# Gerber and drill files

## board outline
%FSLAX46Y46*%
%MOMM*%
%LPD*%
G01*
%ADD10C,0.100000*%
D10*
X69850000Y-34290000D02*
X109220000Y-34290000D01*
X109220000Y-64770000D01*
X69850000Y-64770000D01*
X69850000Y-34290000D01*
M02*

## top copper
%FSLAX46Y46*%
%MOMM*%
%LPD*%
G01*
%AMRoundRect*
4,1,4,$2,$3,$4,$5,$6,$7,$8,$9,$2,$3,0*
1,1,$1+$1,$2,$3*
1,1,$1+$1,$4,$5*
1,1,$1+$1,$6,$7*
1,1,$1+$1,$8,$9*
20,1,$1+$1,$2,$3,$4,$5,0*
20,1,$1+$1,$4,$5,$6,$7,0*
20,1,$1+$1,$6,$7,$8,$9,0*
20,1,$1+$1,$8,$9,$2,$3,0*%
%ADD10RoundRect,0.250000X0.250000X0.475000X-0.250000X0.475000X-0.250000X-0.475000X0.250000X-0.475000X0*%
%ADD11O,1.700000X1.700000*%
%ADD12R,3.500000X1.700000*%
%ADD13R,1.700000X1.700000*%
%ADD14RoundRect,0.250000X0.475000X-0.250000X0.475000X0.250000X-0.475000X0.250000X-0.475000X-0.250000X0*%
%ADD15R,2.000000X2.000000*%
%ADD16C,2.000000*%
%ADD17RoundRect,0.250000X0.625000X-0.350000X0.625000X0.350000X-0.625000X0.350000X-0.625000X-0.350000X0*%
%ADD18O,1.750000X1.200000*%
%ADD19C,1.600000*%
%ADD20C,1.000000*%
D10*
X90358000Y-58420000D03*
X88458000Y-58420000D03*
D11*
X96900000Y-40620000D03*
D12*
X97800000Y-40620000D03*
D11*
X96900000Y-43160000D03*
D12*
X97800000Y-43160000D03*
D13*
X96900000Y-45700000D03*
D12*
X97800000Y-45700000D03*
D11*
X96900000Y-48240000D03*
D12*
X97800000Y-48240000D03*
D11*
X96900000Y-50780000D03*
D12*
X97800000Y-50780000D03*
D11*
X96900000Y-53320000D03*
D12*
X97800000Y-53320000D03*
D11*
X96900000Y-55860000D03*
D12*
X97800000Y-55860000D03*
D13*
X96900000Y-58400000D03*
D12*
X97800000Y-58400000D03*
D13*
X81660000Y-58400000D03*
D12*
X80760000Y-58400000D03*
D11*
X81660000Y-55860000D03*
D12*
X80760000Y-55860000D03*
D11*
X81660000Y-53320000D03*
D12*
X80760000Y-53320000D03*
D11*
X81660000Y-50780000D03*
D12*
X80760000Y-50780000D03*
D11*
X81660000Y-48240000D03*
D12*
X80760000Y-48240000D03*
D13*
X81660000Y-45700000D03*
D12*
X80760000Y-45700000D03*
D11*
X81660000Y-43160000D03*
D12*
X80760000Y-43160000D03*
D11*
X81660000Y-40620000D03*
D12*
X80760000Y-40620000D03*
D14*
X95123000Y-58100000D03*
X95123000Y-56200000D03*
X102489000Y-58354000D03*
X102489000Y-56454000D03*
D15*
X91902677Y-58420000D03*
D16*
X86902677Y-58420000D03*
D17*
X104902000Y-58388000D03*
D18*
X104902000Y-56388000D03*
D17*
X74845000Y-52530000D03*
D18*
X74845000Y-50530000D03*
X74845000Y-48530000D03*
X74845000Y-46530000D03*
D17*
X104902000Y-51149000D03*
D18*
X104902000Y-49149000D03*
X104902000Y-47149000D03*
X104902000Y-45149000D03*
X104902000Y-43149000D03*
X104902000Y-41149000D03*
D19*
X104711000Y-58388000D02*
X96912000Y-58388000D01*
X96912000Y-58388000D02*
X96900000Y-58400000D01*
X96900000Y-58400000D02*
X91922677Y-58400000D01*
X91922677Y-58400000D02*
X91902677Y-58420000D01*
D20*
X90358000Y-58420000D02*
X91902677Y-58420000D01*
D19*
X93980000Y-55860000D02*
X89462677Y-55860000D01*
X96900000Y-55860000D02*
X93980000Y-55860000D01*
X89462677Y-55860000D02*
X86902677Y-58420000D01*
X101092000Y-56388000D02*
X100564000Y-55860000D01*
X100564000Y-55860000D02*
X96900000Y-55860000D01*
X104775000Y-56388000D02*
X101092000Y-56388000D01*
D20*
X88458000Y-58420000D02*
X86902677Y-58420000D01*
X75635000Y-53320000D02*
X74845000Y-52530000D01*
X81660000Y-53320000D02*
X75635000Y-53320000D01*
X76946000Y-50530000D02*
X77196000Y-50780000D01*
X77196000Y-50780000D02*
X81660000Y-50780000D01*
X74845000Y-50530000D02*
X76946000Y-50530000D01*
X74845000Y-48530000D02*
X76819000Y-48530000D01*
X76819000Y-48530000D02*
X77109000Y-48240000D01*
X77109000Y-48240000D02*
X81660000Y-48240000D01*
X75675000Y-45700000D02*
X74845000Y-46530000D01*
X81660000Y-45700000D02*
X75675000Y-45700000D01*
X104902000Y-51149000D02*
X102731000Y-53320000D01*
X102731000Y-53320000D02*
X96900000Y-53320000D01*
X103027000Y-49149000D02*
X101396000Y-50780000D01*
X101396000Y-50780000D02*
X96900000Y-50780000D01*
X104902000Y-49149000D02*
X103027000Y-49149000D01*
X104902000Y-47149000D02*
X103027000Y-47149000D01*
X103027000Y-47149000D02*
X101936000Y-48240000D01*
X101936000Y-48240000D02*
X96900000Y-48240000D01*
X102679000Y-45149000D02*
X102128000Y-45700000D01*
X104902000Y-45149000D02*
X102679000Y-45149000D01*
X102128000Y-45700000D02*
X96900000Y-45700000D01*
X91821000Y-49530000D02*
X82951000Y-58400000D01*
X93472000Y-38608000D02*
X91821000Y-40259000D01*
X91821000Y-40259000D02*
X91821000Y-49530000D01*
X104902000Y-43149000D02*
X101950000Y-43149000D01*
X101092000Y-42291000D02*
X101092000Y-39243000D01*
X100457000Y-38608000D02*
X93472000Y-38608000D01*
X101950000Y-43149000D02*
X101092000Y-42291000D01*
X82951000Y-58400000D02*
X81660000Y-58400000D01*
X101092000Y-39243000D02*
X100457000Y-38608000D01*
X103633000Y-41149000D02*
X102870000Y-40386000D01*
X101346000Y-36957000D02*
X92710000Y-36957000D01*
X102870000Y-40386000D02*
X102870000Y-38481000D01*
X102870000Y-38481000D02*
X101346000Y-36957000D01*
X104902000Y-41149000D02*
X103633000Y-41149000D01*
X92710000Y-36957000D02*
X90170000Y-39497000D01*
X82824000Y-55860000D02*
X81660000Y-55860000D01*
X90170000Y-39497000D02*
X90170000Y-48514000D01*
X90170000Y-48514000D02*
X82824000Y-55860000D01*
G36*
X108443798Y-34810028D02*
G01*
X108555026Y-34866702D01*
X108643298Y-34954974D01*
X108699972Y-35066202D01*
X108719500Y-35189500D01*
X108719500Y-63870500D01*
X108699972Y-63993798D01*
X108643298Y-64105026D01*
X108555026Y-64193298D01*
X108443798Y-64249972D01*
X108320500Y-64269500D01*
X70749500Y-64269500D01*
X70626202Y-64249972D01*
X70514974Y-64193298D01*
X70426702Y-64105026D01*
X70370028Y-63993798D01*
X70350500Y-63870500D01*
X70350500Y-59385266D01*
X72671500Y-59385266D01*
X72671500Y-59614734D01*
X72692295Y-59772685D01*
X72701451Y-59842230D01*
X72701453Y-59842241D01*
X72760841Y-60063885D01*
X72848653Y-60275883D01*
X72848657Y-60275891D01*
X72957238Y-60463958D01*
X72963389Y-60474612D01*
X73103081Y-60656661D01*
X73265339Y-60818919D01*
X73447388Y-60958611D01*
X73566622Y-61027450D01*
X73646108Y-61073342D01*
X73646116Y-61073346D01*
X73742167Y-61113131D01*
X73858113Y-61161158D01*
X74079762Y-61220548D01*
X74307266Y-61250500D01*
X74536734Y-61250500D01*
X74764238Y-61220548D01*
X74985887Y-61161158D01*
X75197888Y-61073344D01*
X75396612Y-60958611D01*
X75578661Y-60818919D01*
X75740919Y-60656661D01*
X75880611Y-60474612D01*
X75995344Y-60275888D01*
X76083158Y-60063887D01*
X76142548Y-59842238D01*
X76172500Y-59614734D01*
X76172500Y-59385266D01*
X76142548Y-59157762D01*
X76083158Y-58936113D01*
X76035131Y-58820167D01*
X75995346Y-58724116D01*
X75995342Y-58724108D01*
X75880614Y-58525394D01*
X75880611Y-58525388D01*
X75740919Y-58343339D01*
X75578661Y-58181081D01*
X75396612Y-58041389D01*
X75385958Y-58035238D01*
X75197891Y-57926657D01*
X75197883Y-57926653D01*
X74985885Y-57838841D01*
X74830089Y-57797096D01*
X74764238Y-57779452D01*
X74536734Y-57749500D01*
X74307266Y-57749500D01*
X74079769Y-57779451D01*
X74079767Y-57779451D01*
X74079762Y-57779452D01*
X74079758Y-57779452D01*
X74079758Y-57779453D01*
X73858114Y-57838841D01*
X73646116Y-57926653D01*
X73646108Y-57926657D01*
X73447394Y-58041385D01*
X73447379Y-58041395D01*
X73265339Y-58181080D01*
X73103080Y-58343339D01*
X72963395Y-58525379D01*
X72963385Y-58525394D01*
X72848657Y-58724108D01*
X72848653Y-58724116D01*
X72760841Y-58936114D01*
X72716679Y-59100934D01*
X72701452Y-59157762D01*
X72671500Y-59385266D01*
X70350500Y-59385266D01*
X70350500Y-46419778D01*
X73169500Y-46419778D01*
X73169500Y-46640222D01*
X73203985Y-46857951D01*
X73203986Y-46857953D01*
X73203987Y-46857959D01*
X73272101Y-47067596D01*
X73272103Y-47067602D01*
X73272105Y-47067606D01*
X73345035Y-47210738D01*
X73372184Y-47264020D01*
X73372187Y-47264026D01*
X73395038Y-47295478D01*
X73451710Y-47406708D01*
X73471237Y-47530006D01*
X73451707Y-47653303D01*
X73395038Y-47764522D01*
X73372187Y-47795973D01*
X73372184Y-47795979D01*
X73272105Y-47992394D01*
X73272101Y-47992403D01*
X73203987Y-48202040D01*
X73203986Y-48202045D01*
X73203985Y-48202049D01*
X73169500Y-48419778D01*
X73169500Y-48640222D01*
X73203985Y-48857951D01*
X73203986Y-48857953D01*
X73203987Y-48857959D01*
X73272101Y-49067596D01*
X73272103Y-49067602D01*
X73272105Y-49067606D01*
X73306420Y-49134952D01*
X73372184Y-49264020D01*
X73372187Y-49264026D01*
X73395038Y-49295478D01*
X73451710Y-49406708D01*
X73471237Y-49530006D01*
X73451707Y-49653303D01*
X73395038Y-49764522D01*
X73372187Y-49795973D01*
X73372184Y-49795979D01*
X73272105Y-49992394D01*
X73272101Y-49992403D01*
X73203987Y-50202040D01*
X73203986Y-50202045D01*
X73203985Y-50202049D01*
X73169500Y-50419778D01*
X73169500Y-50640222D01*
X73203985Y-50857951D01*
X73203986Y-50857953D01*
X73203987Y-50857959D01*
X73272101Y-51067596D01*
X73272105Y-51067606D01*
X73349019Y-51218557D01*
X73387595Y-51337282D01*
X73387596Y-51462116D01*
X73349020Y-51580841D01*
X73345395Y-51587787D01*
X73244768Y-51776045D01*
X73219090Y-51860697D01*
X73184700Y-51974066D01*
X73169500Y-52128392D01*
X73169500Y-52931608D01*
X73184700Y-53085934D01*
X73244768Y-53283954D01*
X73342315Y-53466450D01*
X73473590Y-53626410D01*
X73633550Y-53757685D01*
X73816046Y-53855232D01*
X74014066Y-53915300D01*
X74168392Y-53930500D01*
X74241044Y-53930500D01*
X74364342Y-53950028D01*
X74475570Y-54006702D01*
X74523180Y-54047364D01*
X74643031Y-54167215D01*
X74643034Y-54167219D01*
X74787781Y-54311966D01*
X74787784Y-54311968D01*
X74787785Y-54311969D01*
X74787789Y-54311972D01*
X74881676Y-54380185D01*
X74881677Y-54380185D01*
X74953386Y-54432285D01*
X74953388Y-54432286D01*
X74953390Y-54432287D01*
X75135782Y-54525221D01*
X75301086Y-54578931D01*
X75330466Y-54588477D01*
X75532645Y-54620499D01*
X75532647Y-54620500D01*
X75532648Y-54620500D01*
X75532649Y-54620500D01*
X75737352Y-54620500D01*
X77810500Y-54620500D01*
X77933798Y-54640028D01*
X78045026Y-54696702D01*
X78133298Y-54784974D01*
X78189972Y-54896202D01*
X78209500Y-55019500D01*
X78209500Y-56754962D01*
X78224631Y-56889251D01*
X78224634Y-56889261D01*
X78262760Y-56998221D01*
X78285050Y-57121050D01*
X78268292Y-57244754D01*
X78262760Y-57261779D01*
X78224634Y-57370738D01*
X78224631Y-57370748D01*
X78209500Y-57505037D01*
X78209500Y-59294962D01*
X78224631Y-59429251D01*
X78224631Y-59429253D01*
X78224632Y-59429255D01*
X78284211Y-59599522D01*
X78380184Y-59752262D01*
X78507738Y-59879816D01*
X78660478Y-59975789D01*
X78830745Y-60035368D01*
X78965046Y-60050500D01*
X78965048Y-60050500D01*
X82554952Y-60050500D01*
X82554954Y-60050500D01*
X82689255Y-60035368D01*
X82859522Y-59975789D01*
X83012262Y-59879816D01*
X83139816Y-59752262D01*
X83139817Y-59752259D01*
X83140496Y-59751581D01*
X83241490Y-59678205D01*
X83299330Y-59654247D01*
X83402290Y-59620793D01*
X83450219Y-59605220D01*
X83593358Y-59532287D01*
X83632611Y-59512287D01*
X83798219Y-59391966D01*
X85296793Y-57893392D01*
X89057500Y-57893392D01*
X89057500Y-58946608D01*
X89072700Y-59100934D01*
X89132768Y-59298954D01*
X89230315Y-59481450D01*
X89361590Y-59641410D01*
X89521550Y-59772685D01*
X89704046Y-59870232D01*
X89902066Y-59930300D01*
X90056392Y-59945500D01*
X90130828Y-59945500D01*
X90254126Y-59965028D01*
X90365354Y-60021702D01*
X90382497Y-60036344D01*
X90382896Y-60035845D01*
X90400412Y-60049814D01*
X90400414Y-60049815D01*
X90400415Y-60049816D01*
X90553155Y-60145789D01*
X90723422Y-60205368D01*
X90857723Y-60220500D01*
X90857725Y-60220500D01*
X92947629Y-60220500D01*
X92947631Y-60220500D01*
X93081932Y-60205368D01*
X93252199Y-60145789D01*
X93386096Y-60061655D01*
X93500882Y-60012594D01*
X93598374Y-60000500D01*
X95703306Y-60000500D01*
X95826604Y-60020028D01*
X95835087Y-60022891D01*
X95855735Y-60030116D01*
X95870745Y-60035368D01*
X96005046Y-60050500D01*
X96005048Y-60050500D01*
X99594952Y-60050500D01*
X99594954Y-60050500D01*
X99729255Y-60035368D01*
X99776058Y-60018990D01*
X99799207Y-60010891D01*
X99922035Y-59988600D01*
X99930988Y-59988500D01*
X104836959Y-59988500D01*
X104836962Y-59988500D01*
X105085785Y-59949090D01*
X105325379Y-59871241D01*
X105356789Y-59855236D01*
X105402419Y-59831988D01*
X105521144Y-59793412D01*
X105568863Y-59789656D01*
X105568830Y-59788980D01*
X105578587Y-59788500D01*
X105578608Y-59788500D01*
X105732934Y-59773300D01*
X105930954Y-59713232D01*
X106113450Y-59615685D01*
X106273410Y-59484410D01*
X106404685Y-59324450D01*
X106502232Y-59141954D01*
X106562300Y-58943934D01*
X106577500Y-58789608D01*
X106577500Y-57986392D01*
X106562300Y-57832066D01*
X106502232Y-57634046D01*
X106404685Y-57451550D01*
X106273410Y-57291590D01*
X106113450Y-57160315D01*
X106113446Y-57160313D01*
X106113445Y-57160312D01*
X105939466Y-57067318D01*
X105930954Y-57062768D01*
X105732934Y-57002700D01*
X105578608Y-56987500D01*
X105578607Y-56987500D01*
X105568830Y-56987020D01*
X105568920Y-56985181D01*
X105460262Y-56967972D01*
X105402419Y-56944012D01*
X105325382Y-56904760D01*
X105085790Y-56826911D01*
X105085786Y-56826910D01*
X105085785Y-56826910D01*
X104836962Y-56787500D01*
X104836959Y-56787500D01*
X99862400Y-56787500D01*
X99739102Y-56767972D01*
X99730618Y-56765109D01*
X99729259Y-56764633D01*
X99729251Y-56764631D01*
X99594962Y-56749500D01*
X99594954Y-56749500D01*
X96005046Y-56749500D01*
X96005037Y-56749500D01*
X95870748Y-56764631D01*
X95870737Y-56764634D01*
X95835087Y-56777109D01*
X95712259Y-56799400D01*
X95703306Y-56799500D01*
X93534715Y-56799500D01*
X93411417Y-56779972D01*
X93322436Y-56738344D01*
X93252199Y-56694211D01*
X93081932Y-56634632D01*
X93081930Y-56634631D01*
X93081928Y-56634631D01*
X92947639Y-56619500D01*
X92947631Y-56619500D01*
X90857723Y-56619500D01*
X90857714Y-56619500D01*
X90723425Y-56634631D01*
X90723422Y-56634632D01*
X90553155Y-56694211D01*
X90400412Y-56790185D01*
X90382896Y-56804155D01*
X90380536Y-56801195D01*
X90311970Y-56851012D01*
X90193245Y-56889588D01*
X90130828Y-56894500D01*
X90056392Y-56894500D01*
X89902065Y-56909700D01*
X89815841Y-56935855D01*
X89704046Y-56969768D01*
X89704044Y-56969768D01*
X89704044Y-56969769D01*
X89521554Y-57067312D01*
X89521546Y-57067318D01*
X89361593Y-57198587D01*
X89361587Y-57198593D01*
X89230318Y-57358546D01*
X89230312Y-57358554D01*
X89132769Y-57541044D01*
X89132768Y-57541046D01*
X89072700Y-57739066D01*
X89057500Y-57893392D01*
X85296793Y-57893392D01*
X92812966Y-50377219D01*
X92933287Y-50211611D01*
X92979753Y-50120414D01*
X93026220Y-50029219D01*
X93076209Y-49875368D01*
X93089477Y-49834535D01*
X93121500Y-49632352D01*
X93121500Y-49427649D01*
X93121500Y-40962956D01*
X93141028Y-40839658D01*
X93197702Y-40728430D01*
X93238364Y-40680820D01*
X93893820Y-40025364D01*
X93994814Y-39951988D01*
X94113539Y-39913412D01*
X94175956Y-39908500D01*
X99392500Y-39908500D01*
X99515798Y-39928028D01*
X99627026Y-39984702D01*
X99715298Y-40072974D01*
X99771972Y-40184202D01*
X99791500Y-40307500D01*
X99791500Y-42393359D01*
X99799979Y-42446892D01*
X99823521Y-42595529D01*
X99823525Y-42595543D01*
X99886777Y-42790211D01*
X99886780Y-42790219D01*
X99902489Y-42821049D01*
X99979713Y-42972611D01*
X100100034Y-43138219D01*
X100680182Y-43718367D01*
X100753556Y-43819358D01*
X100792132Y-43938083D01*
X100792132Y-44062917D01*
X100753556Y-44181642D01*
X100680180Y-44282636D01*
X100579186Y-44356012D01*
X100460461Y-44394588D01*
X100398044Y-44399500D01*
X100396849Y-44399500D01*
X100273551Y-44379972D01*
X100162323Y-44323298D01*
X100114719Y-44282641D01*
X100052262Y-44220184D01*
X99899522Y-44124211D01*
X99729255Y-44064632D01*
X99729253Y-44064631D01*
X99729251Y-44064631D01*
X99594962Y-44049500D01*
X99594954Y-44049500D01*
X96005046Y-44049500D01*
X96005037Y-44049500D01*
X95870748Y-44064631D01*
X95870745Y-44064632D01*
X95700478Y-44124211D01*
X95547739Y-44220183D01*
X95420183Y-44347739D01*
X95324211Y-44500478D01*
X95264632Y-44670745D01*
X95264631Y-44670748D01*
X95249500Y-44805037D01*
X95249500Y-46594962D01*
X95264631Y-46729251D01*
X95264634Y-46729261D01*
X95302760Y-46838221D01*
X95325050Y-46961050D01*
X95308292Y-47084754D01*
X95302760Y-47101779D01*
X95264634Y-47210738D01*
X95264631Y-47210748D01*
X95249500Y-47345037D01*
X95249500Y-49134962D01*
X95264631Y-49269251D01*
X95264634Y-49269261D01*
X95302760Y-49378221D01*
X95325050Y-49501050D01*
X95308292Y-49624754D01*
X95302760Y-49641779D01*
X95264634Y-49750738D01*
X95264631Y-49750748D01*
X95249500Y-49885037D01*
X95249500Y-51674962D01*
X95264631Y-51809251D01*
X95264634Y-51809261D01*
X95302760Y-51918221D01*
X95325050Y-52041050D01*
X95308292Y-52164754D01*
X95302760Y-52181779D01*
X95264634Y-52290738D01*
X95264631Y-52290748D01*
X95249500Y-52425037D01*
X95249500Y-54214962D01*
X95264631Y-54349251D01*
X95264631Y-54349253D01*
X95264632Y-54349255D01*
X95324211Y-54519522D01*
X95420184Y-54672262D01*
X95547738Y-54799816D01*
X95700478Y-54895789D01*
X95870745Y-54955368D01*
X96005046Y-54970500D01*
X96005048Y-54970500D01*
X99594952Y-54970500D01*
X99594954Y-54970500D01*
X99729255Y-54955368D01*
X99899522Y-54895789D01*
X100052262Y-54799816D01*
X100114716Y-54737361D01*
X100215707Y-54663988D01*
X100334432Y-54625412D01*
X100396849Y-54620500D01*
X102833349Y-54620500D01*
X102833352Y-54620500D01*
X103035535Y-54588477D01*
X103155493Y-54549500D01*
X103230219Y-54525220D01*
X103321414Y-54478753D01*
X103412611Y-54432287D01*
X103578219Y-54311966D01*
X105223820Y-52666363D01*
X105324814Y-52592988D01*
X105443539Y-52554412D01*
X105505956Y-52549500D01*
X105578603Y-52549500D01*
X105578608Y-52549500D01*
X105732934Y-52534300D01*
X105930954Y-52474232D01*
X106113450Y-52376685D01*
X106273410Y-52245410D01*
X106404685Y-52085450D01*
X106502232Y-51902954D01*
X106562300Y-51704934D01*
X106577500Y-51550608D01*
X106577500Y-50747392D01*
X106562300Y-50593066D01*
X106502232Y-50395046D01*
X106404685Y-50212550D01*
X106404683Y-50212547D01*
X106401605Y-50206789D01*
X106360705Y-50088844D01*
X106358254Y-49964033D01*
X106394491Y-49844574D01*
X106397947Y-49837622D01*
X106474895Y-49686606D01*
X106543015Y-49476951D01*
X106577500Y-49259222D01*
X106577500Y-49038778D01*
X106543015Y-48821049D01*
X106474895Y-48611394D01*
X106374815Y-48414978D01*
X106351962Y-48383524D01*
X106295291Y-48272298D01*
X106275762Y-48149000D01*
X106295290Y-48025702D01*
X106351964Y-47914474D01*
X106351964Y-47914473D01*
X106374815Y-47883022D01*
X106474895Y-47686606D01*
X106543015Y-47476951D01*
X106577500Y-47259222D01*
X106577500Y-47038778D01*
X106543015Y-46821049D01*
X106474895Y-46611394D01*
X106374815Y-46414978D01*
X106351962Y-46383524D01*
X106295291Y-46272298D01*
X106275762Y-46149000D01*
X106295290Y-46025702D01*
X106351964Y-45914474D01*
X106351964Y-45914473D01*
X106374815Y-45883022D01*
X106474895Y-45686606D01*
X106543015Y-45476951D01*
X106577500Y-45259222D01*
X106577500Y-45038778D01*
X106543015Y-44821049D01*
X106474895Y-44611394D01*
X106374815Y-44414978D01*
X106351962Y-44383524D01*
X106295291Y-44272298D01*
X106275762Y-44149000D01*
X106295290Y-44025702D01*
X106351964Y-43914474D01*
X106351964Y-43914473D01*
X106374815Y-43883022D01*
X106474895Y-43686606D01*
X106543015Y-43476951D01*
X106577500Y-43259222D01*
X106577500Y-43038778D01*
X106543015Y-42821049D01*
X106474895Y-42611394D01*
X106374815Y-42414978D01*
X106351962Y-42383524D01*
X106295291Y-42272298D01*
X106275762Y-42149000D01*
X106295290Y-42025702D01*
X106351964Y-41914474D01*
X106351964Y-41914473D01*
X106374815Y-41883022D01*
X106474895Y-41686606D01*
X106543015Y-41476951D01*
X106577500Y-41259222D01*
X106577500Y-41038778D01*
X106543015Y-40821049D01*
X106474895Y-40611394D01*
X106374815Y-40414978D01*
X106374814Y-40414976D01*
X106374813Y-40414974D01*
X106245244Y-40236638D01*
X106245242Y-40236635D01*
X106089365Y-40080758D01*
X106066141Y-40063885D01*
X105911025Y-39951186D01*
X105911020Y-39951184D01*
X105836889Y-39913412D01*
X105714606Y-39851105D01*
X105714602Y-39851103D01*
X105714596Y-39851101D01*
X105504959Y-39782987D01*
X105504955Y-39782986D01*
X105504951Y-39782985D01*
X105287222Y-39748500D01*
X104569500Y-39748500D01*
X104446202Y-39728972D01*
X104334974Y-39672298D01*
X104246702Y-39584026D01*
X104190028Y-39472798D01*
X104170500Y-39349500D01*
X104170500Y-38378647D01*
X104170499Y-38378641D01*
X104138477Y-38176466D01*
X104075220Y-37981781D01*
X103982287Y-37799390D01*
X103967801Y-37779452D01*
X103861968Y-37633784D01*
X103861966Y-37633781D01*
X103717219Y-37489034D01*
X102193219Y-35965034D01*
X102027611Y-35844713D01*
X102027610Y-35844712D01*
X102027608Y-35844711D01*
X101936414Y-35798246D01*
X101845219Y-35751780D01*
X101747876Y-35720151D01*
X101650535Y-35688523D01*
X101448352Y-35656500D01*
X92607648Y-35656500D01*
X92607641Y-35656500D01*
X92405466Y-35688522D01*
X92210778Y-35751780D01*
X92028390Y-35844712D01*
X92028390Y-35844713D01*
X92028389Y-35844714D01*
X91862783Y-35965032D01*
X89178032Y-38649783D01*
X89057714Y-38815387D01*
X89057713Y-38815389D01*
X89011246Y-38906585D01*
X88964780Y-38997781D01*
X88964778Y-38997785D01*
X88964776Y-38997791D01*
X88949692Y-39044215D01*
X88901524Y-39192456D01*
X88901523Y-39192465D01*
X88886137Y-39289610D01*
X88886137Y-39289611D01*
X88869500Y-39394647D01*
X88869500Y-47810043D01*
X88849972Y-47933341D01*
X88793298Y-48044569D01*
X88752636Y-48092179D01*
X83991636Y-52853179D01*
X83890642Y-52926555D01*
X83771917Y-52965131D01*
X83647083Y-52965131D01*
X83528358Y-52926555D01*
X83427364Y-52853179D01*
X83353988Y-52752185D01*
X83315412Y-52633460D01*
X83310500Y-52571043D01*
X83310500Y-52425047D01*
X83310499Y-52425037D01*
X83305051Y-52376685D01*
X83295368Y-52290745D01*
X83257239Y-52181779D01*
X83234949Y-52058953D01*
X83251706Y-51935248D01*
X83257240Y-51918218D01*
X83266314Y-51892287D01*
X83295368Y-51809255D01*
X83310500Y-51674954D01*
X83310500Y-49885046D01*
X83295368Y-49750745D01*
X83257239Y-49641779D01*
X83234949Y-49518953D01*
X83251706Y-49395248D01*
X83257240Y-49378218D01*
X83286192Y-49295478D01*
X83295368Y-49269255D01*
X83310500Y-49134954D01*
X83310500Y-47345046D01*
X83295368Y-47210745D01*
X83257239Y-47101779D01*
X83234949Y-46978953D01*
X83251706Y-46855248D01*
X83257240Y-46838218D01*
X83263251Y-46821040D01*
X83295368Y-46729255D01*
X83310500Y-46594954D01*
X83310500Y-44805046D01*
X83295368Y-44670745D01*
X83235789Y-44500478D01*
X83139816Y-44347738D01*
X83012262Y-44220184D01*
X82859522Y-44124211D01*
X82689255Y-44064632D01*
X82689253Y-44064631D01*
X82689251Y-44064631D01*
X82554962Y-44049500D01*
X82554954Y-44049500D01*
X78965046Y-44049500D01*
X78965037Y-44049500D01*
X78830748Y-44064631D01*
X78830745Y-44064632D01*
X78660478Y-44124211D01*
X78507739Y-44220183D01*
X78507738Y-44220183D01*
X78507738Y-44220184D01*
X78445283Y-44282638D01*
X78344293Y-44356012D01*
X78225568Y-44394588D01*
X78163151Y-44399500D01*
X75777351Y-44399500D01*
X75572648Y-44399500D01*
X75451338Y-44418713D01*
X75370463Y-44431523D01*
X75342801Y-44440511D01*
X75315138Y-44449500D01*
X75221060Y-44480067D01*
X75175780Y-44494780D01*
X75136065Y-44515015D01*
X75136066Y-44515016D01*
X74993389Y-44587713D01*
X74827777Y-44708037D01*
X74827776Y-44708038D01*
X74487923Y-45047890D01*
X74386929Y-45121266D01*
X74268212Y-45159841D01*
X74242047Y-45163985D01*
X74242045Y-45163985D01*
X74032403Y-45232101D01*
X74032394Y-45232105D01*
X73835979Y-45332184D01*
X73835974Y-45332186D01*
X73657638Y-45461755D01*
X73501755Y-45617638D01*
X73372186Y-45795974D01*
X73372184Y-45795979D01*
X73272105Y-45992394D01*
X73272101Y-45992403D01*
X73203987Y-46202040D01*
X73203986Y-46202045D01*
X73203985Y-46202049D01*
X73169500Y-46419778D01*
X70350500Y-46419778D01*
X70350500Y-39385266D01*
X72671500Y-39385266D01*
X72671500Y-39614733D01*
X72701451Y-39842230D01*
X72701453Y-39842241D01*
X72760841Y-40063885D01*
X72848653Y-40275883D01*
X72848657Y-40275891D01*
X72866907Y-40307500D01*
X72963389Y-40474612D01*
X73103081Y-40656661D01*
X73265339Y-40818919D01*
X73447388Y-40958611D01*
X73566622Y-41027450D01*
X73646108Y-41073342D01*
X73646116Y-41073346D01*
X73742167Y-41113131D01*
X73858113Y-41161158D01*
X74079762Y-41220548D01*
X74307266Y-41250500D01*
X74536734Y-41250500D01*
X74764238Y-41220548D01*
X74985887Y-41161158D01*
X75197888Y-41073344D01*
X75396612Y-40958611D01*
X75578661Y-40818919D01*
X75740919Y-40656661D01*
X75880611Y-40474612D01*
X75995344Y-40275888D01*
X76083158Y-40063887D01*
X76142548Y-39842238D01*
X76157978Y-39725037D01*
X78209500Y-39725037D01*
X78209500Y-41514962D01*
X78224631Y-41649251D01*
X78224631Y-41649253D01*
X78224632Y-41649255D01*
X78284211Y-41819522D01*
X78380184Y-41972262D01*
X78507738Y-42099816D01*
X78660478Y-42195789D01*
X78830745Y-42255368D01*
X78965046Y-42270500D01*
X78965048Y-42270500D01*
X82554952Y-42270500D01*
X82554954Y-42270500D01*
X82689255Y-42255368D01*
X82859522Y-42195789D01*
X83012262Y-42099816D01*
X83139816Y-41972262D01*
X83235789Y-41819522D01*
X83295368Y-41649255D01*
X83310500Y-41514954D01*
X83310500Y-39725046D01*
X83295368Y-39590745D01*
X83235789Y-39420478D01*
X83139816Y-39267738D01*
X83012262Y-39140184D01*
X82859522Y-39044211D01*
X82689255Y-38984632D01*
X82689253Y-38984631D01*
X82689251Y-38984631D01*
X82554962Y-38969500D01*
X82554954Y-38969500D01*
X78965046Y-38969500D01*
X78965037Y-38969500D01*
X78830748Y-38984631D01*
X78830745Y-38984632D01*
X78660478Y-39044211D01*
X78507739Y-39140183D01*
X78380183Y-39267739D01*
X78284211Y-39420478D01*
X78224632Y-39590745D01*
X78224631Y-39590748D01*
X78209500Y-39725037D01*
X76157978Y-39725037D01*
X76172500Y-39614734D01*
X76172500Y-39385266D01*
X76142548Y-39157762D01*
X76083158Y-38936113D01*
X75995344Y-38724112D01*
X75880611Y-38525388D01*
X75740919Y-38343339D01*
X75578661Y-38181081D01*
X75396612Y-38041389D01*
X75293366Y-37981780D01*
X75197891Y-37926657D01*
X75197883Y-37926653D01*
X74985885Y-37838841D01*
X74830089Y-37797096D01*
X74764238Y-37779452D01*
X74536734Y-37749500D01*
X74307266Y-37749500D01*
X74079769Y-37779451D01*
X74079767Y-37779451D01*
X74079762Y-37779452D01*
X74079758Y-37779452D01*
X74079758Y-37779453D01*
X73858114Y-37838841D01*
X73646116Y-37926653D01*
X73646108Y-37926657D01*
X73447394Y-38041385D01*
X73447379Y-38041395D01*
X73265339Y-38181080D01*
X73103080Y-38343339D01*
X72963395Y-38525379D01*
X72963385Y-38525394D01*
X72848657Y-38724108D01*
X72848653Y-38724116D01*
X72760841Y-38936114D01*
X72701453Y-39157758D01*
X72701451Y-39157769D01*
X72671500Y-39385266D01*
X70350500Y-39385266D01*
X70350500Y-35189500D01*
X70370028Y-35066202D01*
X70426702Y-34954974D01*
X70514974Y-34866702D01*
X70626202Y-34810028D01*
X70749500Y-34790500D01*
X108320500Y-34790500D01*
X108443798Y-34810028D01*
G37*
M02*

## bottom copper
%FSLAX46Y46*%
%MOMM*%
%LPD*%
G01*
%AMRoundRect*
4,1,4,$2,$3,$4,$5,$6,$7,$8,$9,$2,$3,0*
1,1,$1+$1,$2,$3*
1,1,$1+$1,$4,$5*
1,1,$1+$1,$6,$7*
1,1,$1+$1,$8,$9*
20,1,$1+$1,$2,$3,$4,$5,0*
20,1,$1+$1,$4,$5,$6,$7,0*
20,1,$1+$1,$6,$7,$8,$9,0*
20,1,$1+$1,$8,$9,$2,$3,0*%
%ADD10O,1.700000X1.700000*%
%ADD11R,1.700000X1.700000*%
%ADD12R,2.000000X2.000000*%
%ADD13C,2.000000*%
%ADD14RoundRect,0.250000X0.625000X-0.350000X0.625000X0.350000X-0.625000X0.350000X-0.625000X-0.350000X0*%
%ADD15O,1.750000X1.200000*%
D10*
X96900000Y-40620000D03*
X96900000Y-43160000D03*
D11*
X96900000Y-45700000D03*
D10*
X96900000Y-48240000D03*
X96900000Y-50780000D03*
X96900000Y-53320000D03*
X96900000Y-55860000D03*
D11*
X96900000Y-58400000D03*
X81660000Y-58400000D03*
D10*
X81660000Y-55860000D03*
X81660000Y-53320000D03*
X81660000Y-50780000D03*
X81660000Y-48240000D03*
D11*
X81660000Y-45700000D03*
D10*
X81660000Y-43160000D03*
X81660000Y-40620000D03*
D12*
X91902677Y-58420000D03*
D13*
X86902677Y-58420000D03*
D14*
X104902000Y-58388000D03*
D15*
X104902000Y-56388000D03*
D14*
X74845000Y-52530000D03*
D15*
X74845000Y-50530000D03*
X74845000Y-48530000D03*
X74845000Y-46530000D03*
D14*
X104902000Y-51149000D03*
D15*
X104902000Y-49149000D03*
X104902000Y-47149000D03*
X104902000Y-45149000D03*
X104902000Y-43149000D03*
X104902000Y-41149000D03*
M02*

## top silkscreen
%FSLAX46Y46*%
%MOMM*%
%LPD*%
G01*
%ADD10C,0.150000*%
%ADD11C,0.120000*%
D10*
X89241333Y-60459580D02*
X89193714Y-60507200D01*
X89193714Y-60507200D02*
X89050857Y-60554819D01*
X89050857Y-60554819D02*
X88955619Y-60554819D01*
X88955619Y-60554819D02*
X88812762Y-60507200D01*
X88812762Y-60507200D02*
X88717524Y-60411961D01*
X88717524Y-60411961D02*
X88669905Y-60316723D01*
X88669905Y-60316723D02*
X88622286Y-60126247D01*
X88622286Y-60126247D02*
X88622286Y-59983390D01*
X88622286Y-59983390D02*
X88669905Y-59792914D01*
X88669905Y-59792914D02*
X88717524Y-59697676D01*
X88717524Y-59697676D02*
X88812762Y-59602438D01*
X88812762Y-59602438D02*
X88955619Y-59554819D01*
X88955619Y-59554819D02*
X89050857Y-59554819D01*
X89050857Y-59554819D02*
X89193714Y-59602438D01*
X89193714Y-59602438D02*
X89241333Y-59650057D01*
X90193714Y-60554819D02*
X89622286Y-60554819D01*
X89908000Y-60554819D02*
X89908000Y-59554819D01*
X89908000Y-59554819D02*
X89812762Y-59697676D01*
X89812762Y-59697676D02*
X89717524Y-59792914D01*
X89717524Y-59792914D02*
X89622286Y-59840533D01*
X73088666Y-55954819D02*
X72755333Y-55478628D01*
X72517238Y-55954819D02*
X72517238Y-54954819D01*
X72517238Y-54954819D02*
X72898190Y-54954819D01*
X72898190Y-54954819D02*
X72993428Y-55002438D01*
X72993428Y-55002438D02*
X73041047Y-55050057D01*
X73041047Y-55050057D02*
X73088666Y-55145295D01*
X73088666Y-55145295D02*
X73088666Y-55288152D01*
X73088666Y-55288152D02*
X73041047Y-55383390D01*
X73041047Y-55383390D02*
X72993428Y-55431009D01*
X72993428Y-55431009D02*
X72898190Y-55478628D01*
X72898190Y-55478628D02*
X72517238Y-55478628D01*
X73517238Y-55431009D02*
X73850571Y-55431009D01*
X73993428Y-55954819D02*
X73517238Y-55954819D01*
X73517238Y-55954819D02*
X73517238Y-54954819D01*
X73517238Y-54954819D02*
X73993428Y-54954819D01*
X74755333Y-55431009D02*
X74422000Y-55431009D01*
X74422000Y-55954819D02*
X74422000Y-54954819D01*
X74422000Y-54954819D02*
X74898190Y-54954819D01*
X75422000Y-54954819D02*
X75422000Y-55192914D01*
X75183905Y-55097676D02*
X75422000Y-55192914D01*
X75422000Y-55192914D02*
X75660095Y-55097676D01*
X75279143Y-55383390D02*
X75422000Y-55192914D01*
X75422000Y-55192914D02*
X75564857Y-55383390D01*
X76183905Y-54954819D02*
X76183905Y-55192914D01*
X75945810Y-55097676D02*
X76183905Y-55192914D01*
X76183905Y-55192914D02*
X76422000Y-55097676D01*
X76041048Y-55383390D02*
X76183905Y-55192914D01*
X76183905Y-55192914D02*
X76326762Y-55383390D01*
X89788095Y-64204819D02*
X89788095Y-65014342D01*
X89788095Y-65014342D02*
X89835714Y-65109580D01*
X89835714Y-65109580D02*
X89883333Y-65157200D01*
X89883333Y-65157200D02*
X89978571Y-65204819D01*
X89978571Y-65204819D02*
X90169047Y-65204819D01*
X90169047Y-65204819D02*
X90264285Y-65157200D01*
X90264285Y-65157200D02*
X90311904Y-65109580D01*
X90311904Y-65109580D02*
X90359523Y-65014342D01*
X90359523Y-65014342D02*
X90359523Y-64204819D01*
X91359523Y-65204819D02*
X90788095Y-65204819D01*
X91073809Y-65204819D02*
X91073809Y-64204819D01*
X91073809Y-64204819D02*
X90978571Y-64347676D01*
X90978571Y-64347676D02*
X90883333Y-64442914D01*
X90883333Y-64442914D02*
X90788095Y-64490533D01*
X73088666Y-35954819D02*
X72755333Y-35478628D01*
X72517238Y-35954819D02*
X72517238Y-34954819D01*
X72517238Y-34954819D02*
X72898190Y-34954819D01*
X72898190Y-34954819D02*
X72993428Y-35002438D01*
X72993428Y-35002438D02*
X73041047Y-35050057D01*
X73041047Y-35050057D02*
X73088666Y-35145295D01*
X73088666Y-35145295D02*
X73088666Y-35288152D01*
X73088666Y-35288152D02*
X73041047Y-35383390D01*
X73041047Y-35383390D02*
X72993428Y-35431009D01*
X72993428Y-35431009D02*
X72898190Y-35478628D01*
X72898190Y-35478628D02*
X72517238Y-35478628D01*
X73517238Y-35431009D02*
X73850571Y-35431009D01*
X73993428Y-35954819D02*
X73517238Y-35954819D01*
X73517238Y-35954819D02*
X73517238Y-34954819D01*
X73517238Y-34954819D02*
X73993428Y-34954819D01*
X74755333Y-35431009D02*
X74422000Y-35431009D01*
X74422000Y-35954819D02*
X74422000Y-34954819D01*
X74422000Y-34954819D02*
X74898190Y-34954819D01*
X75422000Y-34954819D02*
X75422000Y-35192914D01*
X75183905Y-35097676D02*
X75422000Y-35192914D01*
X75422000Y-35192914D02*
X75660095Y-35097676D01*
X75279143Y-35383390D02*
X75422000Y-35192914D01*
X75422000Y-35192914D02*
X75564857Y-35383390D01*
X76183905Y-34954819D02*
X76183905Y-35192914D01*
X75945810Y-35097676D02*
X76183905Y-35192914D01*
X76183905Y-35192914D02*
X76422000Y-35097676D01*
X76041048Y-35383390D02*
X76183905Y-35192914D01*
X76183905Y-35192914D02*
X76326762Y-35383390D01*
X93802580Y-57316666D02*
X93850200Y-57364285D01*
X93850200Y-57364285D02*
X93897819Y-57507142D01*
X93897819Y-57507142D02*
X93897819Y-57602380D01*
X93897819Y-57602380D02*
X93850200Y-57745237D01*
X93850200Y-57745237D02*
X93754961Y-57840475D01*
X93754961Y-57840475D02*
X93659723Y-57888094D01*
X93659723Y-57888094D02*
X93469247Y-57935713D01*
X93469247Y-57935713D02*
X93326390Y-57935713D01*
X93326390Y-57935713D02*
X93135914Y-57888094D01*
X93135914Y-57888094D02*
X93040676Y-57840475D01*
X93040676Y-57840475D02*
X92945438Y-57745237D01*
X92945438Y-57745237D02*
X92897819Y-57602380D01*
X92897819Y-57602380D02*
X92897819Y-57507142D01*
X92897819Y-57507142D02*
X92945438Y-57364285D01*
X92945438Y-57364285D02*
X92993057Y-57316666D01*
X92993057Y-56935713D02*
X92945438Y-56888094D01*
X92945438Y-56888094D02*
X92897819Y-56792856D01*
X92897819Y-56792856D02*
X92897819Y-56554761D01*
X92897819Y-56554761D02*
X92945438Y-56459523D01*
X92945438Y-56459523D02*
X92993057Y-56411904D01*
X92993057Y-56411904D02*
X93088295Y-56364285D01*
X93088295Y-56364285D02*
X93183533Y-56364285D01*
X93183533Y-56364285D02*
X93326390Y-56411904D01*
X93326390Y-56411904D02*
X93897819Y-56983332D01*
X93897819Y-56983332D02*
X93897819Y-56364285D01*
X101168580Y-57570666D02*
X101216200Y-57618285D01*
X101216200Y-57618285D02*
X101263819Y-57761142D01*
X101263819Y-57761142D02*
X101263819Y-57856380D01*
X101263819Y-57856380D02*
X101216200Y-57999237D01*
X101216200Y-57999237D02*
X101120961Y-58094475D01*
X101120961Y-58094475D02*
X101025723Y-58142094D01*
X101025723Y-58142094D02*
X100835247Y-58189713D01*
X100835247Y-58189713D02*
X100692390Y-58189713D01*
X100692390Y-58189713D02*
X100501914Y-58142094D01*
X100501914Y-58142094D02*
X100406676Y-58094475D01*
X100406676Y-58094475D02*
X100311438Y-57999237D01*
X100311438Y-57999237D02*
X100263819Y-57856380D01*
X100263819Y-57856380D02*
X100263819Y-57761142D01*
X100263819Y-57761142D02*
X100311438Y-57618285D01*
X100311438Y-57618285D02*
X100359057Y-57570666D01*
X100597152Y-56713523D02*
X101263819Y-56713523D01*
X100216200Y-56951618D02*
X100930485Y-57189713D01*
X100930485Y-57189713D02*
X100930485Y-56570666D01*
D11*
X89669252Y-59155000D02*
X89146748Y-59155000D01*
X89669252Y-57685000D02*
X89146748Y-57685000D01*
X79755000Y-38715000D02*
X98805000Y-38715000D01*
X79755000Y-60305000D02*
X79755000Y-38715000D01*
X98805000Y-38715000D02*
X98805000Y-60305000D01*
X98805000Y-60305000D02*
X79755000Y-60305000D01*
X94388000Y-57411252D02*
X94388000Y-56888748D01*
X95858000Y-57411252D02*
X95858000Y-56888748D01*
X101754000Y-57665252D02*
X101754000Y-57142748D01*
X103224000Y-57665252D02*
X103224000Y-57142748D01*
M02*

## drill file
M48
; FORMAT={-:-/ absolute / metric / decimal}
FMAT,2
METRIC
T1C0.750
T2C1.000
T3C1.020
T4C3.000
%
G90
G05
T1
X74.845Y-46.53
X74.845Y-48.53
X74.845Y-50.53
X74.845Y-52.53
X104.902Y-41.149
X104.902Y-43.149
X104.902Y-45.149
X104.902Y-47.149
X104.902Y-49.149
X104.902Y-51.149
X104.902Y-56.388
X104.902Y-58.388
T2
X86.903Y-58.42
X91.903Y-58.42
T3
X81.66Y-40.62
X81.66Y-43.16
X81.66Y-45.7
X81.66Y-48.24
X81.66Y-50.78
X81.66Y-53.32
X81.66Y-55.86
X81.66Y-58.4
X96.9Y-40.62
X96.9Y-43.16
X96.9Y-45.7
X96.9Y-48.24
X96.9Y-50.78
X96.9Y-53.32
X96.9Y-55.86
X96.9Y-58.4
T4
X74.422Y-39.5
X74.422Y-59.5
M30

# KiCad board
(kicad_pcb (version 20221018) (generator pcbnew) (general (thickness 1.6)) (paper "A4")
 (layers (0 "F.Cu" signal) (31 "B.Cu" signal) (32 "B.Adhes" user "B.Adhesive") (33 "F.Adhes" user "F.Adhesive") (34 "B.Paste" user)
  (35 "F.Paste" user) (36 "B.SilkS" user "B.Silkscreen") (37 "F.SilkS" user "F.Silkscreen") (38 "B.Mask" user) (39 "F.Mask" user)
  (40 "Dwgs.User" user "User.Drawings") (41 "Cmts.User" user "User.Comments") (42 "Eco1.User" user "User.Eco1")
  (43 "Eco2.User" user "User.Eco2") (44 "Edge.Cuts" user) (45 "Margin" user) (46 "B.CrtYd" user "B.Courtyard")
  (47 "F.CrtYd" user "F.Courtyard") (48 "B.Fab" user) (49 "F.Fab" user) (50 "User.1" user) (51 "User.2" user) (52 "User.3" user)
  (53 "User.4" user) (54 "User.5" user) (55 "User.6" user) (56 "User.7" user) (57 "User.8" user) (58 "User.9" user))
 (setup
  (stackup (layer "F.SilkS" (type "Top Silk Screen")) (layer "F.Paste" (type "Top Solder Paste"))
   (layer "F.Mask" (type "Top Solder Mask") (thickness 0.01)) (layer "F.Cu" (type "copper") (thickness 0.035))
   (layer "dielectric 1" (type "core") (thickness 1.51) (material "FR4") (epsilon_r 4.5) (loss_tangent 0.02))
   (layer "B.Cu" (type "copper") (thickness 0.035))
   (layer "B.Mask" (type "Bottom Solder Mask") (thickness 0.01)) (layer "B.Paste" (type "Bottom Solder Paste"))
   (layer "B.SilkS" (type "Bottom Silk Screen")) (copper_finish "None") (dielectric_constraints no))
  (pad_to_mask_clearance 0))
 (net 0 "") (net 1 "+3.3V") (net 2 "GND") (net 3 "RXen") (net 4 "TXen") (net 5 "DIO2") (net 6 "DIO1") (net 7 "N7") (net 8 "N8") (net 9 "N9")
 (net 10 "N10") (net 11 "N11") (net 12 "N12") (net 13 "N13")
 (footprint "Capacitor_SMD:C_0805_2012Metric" (layer "F.Cu") (at 89.408 58.42 180)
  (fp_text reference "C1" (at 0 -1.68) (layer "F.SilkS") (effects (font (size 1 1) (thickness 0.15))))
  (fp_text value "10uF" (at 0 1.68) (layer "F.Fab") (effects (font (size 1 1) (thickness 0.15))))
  (fp_line (start -0.261252 -0.735) (end 0.261252 -0.735) (stroke (width 0.12) (type solid)) (layer "F.SilkS"))
  (fp_line (start -0.261252 0.735) (end 0.261252 0.735) (stroke (width 0.12) (type solid)) (layer "F.SilkS"))
  (pad "1" smd roundrect (at -0.95 0 180) (size 1 1.45) (layers "F.Cu" "F.Paste" "F.Mask") (roundrect_rratio 0.25) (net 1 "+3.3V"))
  (pad "2" smd roundrect (at 0.95 0 180) (size 1 1.45) (layers "F.Cu" "F.Paste" "F.Mask") (roundrect_rratio 0.25) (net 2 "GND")))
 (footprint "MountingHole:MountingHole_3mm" (layer "F.Cu") (at 74.422 59.5)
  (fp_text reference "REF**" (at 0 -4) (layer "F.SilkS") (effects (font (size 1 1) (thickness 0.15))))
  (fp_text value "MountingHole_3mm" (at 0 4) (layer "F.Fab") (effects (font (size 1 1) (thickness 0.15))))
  (pad "" np_thru_hole circle (at 0 0) (size 3 3) (drill 3) (layers "F&B.Cu" "*.Mask")))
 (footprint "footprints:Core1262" (layer "F.Cu") (at 90.55 64.75)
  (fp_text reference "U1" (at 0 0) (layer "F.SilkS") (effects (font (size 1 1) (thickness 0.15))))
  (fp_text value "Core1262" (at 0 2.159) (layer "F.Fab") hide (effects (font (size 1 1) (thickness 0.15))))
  (fp_line (start -10.795 -26.035) (end 8.255 -26.035) (stroke (width 0.12) (type default)) (layer "F.SilkS"))
  (fp_line (start -10.795 -4.445) (end -10.795 -26.035) (stroke (width 0.12) (type default)) (layer "F.SilkS"))
  (fp_line (start 8.255 -26.035) (end 8.255 -4.445) (stroke (width 0.12) (type default)) (layer "F.SilkS"))
  (fp_line (start 8.255 -4.445) (end -10.795 -4.445) (stroke (width 0.12) (type default)) (layer "F.SilkS"))
  (pad "1" thru_hole oval (at 6.35 -24.13) (size 1.7 1.7) (drill 1.02) (layers "*.Cu" "*.Mask") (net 2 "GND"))
  (pad "1" smd rect (at 6.35 -24.13) (size 3.5 1.7) (drill (offset 0.9 0)) (layers "F.Cu" "F.Mask") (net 2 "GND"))
  (pad "2" thru_hole oval (at 6.35 -21.59) (size 1.7 1.7) (drill 1.02) (layers "*.Cu" "*.Mask") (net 2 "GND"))
  (pad "2" smd rect (at 6.35 -21.59) (size 3.5 1.7) (drill (offset 0.9 0)) (layers "F.Cu" "F.Mask") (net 2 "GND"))
  (pad "3" thru_hole rect (at 6.35 -19.05) (size 1.7 1.7) (drill 1.02) (layers "*.Cu" "*.Mask") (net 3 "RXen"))
  (pad "3" smd rect (at 6.35 -19.05) (size 3.5 1.7) (drill (offset 0.9 0)) (layers "F.Cu" "F.Mask") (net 3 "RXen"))
  (pad "4" thru_hole oval (at 6.35 -16.51) (size 1.7 1.7) (drill 1.02) (layers "*.Cu" "*.Mask") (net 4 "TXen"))
  (pad "4" smd rect (at 6.35 -16.51) (size 3.5 1.7) (drill (offset 0.9 0)) (layers "F.Cu" "F.Mask") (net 4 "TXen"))
  (pad "5" thru_hole oval (at 6.35 -13.97) (size 1.7 1.7) (drill 1.02) (layers "*.Cu" "*.Mask") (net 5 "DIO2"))
  (pad "5" smd rect (at 6.35 -13.97) (size 3.5 1.7) (drill (offset 0.9 0)) (layers "F.Cu" "F.Mask") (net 5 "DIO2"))
  (pad "6" thru_hole oval (at 6.35 -11.43) (size 1.7 1.7) (drill 1.02) (layers "*.Cu" "*.Mask") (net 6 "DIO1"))
  (pad "6" smd rect (at 6.35 -11.43) (size 3.5 1.7) (drill (offset 0.9 0)) (layers "F.Cu" "F.Mask") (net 6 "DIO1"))
  (pad "7" thru_hole oval (at 6.35 -8.89) (size 1.7 1.7) (drill 1.02) (layers "*.Cu" "*.Mask") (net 2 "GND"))
  (pad "7" smd rect (at 6.35 -8.89) (size 3.5 1.7) (drill (offset 0.9 0)) (layers "F.Cu" "F.Mask") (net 2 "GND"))
  (pad "8" thru_hole rect (at 6.35 -6.35) (size 1.7 1.7) (drill 1.02) (layers "*.Cu" "*.Mask") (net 1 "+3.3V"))
  (pad "8" smd rect (at 6.35 -6.35) (size 3.5 1.7) (drill (offset 0.9 0)) (layers "F.Cu" "F.Mask") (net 1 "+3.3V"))
  (pad "9" thru_hole rect (at -8.89 -6.35) (size 1.7 1.7) (drill 1.02) (layers "*.Cu" "*.Mask") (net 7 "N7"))
  (pad "9" smd rect (at -8.89 -6.35) (size 3.5 1.7) (drill (offset -0.9 0)) (layers "F.Cu" "F.Mask") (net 7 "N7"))
  (pad "10" thru_hole oval (at -8.89 -8.89) (size 1.7 1.7) (drill 1.02) (layers "*.Cu" "*.Mask") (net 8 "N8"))
  (pad "10" smd rect (at -8.89 -8.89) (size 3.5 1.7) (drill (offset -0.9 0)) (layers "F.Cu" "F.Mask") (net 8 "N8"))
  (pad "11" thru_hole oval (at -8.89 -11.43) (size 1.7 1.7) (drill 1.02) (layers "*.Cu" "*.Mask") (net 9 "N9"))
  (pad "11" smd rect (at -8.89 -11.43) (size 3.5 1.7) (drill (offset -0.9 0)) (layers "F.Cu" "F.Mask") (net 9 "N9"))
  (pad "12" thru_hole oval (at -8.89 -13.97) (size 1.7 1.7) (drill 1.02) (layers "*.Cu" "*.Mask") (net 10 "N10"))
  (pad "12" smd rect (at -8.89 -13.97) (size 3.5 1.7) (drill (offset -0.9 0)) (layers "F.Cu" "F.Mask") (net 10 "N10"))
  (pad "13" thru_hole oval (at -8.89 -16.51) (size 1.7 1.7) (drill 1.02) (layers "*.Cu" "*.Mask") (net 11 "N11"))
  (pad "13" smd rect (at -8.89 -16.51) (size 3.5 1.7) (drill (offset -0.9 0)) (layers "F.Cu" "F.Mask") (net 11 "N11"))
  (pad "14" thru_hole rect (at -8.89 -19.05) (size 1.7 1.7) (drill 1.02) (layers "*.Cu" "*.Mask") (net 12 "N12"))
  (pad "14" smd rect (at -8.89 -19.05) (size 3.5 1.7) (drill (offset -0.9 0)) (layers "F.Cu" "F.Mask") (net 12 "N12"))
  (pad "15" thru_hole oval (at -8.89 -21.59) (size 1.7 1.7) (drill 1.02) (layers "*.Cu" "*.Mask") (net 2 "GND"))
  (pad "15" smd rect (at -8.89 -21.59) (size 3.5 1.7) (drill (offset -0.9 0)) (layers "F.Cu" "F.Mask") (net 2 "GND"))
  (pad "16" thru_hole oval (at -8.89 -24.13) (size 1.7 1.7) (drill 1.02) (layers "*.Cu" "*.Mask") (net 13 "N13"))
  (pad "16" smd rect (at -8.89 -24.13) (size 3.5 1.7) (drill (offset -0.9 0)) (layers "F.Cu" "F.Mask") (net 13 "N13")))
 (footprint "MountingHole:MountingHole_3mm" (layer "F.Cu") (at 74.422 39.5)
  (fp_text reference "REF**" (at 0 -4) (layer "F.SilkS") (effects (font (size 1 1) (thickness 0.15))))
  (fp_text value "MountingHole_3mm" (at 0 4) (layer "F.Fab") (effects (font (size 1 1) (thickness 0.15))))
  (pad "" np_thru_hole circle (at 0 0) (size 3 3) (drill 3) (layers "*.Cu" "*.Mask")))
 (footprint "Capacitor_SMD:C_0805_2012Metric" (layer "F.Cu") (at 95.123 57.15 90)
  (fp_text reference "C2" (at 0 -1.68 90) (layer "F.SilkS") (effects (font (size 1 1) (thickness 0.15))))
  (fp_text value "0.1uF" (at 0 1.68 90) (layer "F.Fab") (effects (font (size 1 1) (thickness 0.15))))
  (fp_line (start -0.261252 -0.735) (end 0.261252 -0.735) (stroke (width 0.12) (type solid)) (layer "F.SilkS"))
  (fp_line (start -0.261252 0.735) (end 0.261252 0.735) (stroke (width 0.12) (type solid)) (layer "F.SilkS"))
  (pad "1" smd roundrect (at -0.95 0 90) (size 1 1.45) (layers "F.Cu" "F.Paste" "F.Mask") (roundrect_rratio 0.25) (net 1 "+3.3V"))
  (pad "2" smd roundrect (at 0.95 0 90) (size 1 1.45) (layers "F.Cu" "F.Paste" "F.Mask") (roundrect_rratio 0.25) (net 2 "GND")))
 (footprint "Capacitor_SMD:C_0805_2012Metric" (layer "F.Cu") (at 102.489 57.404 90)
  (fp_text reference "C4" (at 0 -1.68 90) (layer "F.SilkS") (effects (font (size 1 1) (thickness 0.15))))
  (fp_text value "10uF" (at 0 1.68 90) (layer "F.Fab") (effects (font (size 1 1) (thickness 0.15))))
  (fp_line (start -0.261252 -0.735) (end 0.261252 -0.735) (stroke (width 0.12) (type solid)) (layer "F.SilkS"))
  (fp_line (start -0.261252 0.735) (end 0.261252 0.735) (stroke (width 0.12) (type solid)) (layer "F.SilkS"))
  (pad "1" smd roundrect (at -0.95 0 90) (size 1 1.45) (layers "F.Cu" "F.Paste" "F.Mask") (roundrect_rratio 0.25) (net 1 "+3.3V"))
  (pad "2" smd roundrect (at 0.95 0 90) (size 1 1.45) (layers "F.Cu" "F.Paste" "F.Mask") (roundrect_rratio 0.25) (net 2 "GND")))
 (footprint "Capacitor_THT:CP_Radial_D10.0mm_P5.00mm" (layer "B.Cu") (at 91.902677 58.42 180)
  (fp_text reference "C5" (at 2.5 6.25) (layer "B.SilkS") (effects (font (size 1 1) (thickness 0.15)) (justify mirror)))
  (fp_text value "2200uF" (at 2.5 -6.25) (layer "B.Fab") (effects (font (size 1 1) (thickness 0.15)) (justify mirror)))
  (pad "1" thru_hole rect (at 0 0 180) (size 2 2) (drill 1) (layers "*.Cu" "*.Mask") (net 1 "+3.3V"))
  (pad "2" thru_hole circle (at 5 0 180) (size 2 2) (drill 1) (layers "*.Cu" "*.Mask") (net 2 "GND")))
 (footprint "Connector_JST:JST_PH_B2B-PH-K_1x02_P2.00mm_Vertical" (layer "B.Cu") (at 104.902 58.388 90)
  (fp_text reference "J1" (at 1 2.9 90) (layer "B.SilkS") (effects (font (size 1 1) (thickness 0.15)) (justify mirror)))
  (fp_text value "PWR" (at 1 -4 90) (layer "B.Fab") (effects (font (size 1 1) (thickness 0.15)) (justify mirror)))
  (pad "1" thru_hole roundrect (at 0 0 90) (size 1.2 1.75) (drill 0.75) (layers "*.Cu" "*.Mask") (roundrect_rratio 0.208333) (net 1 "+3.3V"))
  (pad "2" thru_hole oval (at 2 0 90) (size 1.2 1.75) (drill 0.75) (layers "*.Cu" "*.Mask") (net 2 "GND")))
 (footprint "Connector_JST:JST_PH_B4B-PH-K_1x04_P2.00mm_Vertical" (layer "B.Cu") (at 74.845 52.53 90)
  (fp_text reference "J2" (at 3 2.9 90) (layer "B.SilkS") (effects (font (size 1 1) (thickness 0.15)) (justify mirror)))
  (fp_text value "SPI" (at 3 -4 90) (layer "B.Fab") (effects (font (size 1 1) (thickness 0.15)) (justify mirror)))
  (pad "1" thru_hole roundrect (at 0 0 90) (size 1.2 1.75) (drill 0.75) (layers "*.Cu" "*.Mask") (roundrect_rratio 0.208333) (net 9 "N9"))
  (pad "2" thru_hole oval (at 2 0 90) (size 1.2 1.75) (drill 0.75) (layers "*.Cu" "*.Mask") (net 10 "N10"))
  (pad "3" thru_hole oval (at 4 0 90) (size 1.2 1.75) (drill 0.75) (layers "*.Cu" "*.Mask") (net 11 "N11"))
  (pad "4" thru_hole oval (at 6 0 90) (size 1.2 1.75) (drill 0.75) (layers "*.Cu" "*.Mask") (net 12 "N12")))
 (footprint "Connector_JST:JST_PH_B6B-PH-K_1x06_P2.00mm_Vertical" (layer "B.Cu") (at 104.902 51.149 90)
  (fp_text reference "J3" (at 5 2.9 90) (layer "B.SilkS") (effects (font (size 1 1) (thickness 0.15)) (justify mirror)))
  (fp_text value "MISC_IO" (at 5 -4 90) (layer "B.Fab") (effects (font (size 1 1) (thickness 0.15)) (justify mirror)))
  (pad "1" thru_hole roundrect (at 0 0 90) (size 1.2 1.75) (drill 0.75) (layers "*.Cu" "*.Mask") (roundrect_rratio 0.208333) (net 6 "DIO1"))
  (pad "2" thru_hole oval (at 2 0 90) (size 1.2 1.75) (drill 0.75) (layers "*.Cu" "*.Mask") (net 5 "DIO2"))
  (pad "3" thru_hole oval (at 4 0 90) (size 1.2 1.75) (drill 0.75) (layers "*.Cu" "*.Mask") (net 4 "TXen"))
  (pad "4" thru_hole oval (at 6 0 90) (size 1.2 1.75) (drill 0.75) (layers "*.Cu" "*.Mask") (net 3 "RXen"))
  (pad "5" thru_hole oval (at 8 0 90) (size 1.2 1.75) (drill 0.75) (layers "*.Cu" "*.Mask") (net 7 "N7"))
  (pad "6" thru_hole oval (at 10 0 90) (size 1.2 1.75) (drill 0.75) (layers "*.Cu" "*.Mask") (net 8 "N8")))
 (gr_rect (start 69.85 34.29) (end 109.22 64.77) (stroke (width 0.1) (type default)) (fill none) (layer "Edge.Cuts"))
 (segment (start 104.711 58.388) (end 96.912 58.388) (width 1.6) (layer "F.Cu") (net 1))
 (segment (start 96.912 58.388) (end 96.9 58.4) (width 1.6) (layer "F.Cu") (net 1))
 (segment (start 96.9 58.4) (end 91.922677 58.4) (width 1.6) (layer "F.Cu") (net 1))
 (segment (start 91.922677 58.4) (end 91.902677 58.42) (width 1.6) (layer "F.Cu") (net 1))
 (segment (start 90.358 58.42) (end 91.902677 58.42) (width 1) (layer "F.Cu") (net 1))
 (segment (start 93.98 55.86) (end 89.462677 55.86) (width 1.6) (layer "F.Cu") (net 2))
 (segment (start 96.9 55.86) (end 93.98 55.86) (width 1.6) (layer "F.Cu") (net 2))
 (segment (start 89.462677 55.86) (end 86.902677 58.42) (width 1.6) (layer "F.Cu") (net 2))
 (segment (start 101.092 56.388) (end 100.564 55.86) (width 1.6) (layer "F.Cu") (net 2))
 (segment (start 100.564 55.86) (end 96.9 55.86) (width 1.6) (layer "F.Cu") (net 2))
 (segment (start 104.775 56.388) (end 101.092 56.388) (width 1.6) (layer "F.Cu") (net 2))
 (segment (start 88.458 58.42) (end 86.902677 58.42) (width 1) (layer "F.Cu") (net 2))
 (segment (start 75.635 53.32) (end 74.845 52.53) (width 1) (layer "F.Cu") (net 9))
 (segment (start 81.66 53.32) (end 75.635 53.32) (width 1) (layer "F.Cu") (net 9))
 (segment (start 76.946 50.53) (end 77.196 50.78) (width 1) (layer "F.Cu") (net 10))
 (segment (start 77.196 50.78) (end 81.66 50.78) (width 1) (layer "F.Cu") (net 10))
 (segment (start 74.845 50.53) (end 76.946 50.53) (width 1) (layer "F.Cu") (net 10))
 (segment (start 74.845 48.53) (end 76.819 48.53) (width 1) (layer "F.Cu") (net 11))
 (segment (start 76.819 48.53) (end 77.109 48.24) (width 1) (layer "F.Cu") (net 11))
 (segment (start 77.109 48.24) (end 81.66 48.24) (width 1) (layer "F.Cu") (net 11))
 (segment (start 75.675 45.7) (end 74.845 46.53) (width 1) (layer "F.Cu") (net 12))
 (segment (start 81.66 45.7) (end 75.675 45.7) (width 1) (layer "F.Cu") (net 12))
 (segment (start 104.902 51.149) (end 102.731 53.32) (width 1) (layer "F.Cu") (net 6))
 (segment (start 102.731 53.32) (end 96.9 53.32) (width 1) (layer "F.Cu") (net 6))
 (segment (start 103.027 49.149) (end 101.396 50.78) (width 1) (layer "F.Cu") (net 5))
 (segment (start 101.396 50.78) (end 96.9 50.78) (width 1) (layer "F.Cu") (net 5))
 (segment (start 104.902 49.149) (end 103.027 49.149) (width 1) (layer "F.Cu") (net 5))
 (segment (start 104.902 47.149) (end 103.027 47.149) (width 1) (layer "F.Cu") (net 4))
 (segment (start 103.027 47.149) (end 101.936 48.24) (width 1) (layer "F.Cu") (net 4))
 (segment (start 101.936 48.24) (end 96.9 48.24) (width 1) (layer "F.Cu") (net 4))
 (segment (start 102.679 45.149) (end 102.128 45.7) (width 1) (layer "F.Cu") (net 3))
 (segment (start 104.902 45.149) (end 102.679 45.149) (width 1) (layer "F.Cu") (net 3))
 (segment (start 102.128 45.7) (end 96.9 45.7) (width 1) (layer "F.Cu") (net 3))
 (segment (start 91.821 49.53) (end 82.951 58.4) (width 1) (layer "F.Cu") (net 7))
 (segment (start 93.472 38.608) (end 91.821 40.259) (width 1) (layer "F.Cu") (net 7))
 (segment (start 91.821 40.259) (end 91.821 49.53) (width 1) (layer "F.Cu") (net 7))
 (segment (start 104.902 43.149) (end 101.95 43.149) (width 1) (layer "F.Cu") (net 7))
 (segment (start 101.092 42.291) (end 101.092 39.243) (width 1) (layer "F.Cu") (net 7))
 (segment (start 100.457 38.608) (end 93.472 38.608) (width 1) (layer "F.Cu") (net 7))
 (segment (start 101.95 43.149) (end 101.092 42.291) (width 1) (layer "F.Cu") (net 7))
 (segment (start 82.951 58.4) (end 81.66 58.4) (width 1) (layer "F.Cu") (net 7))
 (segment (start 101.092 39.243) (end 100.457 38.608) (width 1) (layer "F.Cu") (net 7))
 (segment (start 103.633 41.149) (end 102.87 40.386) (width 1) (layer "F.Cu") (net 8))
 (segment (start 101.346 36.957) (end 92.71 36.957) (width 1) (layer "F.Cu") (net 8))
 (segment (start 102.87 40.386) (end 102.87 38.481) (width 1) (layer "F.Cu") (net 8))
 (segment (start 102.87 38.481) (end 101.346 36.957) (width 1) (layer "F.Cu") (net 8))
 (segment (start 104.902 41.149) (end 103.633 41.149) (width 1) (layer "F.Cu") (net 8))
 (segment (start 92.71 36.957) (end 90.17 39.497) (width 1) (layer "F.Cu") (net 8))
 (segment (start 82.824 55.86) (end 81.66 55.86) (width 1) (layer "F.Cu") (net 8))
 (segment (start 90.17 39.497) (end 90.17 48.514) (width 1) (layer "F.Cu") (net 8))
 (segment (start 90.17 48.514) (end 82.824 55.86) (width 1) (layer "F.Cu") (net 8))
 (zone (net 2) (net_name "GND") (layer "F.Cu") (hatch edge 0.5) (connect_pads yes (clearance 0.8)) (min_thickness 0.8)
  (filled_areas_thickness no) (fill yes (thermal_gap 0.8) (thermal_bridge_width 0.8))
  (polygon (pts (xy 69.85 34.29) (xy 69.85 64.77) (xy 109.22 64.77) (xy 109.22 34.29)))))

